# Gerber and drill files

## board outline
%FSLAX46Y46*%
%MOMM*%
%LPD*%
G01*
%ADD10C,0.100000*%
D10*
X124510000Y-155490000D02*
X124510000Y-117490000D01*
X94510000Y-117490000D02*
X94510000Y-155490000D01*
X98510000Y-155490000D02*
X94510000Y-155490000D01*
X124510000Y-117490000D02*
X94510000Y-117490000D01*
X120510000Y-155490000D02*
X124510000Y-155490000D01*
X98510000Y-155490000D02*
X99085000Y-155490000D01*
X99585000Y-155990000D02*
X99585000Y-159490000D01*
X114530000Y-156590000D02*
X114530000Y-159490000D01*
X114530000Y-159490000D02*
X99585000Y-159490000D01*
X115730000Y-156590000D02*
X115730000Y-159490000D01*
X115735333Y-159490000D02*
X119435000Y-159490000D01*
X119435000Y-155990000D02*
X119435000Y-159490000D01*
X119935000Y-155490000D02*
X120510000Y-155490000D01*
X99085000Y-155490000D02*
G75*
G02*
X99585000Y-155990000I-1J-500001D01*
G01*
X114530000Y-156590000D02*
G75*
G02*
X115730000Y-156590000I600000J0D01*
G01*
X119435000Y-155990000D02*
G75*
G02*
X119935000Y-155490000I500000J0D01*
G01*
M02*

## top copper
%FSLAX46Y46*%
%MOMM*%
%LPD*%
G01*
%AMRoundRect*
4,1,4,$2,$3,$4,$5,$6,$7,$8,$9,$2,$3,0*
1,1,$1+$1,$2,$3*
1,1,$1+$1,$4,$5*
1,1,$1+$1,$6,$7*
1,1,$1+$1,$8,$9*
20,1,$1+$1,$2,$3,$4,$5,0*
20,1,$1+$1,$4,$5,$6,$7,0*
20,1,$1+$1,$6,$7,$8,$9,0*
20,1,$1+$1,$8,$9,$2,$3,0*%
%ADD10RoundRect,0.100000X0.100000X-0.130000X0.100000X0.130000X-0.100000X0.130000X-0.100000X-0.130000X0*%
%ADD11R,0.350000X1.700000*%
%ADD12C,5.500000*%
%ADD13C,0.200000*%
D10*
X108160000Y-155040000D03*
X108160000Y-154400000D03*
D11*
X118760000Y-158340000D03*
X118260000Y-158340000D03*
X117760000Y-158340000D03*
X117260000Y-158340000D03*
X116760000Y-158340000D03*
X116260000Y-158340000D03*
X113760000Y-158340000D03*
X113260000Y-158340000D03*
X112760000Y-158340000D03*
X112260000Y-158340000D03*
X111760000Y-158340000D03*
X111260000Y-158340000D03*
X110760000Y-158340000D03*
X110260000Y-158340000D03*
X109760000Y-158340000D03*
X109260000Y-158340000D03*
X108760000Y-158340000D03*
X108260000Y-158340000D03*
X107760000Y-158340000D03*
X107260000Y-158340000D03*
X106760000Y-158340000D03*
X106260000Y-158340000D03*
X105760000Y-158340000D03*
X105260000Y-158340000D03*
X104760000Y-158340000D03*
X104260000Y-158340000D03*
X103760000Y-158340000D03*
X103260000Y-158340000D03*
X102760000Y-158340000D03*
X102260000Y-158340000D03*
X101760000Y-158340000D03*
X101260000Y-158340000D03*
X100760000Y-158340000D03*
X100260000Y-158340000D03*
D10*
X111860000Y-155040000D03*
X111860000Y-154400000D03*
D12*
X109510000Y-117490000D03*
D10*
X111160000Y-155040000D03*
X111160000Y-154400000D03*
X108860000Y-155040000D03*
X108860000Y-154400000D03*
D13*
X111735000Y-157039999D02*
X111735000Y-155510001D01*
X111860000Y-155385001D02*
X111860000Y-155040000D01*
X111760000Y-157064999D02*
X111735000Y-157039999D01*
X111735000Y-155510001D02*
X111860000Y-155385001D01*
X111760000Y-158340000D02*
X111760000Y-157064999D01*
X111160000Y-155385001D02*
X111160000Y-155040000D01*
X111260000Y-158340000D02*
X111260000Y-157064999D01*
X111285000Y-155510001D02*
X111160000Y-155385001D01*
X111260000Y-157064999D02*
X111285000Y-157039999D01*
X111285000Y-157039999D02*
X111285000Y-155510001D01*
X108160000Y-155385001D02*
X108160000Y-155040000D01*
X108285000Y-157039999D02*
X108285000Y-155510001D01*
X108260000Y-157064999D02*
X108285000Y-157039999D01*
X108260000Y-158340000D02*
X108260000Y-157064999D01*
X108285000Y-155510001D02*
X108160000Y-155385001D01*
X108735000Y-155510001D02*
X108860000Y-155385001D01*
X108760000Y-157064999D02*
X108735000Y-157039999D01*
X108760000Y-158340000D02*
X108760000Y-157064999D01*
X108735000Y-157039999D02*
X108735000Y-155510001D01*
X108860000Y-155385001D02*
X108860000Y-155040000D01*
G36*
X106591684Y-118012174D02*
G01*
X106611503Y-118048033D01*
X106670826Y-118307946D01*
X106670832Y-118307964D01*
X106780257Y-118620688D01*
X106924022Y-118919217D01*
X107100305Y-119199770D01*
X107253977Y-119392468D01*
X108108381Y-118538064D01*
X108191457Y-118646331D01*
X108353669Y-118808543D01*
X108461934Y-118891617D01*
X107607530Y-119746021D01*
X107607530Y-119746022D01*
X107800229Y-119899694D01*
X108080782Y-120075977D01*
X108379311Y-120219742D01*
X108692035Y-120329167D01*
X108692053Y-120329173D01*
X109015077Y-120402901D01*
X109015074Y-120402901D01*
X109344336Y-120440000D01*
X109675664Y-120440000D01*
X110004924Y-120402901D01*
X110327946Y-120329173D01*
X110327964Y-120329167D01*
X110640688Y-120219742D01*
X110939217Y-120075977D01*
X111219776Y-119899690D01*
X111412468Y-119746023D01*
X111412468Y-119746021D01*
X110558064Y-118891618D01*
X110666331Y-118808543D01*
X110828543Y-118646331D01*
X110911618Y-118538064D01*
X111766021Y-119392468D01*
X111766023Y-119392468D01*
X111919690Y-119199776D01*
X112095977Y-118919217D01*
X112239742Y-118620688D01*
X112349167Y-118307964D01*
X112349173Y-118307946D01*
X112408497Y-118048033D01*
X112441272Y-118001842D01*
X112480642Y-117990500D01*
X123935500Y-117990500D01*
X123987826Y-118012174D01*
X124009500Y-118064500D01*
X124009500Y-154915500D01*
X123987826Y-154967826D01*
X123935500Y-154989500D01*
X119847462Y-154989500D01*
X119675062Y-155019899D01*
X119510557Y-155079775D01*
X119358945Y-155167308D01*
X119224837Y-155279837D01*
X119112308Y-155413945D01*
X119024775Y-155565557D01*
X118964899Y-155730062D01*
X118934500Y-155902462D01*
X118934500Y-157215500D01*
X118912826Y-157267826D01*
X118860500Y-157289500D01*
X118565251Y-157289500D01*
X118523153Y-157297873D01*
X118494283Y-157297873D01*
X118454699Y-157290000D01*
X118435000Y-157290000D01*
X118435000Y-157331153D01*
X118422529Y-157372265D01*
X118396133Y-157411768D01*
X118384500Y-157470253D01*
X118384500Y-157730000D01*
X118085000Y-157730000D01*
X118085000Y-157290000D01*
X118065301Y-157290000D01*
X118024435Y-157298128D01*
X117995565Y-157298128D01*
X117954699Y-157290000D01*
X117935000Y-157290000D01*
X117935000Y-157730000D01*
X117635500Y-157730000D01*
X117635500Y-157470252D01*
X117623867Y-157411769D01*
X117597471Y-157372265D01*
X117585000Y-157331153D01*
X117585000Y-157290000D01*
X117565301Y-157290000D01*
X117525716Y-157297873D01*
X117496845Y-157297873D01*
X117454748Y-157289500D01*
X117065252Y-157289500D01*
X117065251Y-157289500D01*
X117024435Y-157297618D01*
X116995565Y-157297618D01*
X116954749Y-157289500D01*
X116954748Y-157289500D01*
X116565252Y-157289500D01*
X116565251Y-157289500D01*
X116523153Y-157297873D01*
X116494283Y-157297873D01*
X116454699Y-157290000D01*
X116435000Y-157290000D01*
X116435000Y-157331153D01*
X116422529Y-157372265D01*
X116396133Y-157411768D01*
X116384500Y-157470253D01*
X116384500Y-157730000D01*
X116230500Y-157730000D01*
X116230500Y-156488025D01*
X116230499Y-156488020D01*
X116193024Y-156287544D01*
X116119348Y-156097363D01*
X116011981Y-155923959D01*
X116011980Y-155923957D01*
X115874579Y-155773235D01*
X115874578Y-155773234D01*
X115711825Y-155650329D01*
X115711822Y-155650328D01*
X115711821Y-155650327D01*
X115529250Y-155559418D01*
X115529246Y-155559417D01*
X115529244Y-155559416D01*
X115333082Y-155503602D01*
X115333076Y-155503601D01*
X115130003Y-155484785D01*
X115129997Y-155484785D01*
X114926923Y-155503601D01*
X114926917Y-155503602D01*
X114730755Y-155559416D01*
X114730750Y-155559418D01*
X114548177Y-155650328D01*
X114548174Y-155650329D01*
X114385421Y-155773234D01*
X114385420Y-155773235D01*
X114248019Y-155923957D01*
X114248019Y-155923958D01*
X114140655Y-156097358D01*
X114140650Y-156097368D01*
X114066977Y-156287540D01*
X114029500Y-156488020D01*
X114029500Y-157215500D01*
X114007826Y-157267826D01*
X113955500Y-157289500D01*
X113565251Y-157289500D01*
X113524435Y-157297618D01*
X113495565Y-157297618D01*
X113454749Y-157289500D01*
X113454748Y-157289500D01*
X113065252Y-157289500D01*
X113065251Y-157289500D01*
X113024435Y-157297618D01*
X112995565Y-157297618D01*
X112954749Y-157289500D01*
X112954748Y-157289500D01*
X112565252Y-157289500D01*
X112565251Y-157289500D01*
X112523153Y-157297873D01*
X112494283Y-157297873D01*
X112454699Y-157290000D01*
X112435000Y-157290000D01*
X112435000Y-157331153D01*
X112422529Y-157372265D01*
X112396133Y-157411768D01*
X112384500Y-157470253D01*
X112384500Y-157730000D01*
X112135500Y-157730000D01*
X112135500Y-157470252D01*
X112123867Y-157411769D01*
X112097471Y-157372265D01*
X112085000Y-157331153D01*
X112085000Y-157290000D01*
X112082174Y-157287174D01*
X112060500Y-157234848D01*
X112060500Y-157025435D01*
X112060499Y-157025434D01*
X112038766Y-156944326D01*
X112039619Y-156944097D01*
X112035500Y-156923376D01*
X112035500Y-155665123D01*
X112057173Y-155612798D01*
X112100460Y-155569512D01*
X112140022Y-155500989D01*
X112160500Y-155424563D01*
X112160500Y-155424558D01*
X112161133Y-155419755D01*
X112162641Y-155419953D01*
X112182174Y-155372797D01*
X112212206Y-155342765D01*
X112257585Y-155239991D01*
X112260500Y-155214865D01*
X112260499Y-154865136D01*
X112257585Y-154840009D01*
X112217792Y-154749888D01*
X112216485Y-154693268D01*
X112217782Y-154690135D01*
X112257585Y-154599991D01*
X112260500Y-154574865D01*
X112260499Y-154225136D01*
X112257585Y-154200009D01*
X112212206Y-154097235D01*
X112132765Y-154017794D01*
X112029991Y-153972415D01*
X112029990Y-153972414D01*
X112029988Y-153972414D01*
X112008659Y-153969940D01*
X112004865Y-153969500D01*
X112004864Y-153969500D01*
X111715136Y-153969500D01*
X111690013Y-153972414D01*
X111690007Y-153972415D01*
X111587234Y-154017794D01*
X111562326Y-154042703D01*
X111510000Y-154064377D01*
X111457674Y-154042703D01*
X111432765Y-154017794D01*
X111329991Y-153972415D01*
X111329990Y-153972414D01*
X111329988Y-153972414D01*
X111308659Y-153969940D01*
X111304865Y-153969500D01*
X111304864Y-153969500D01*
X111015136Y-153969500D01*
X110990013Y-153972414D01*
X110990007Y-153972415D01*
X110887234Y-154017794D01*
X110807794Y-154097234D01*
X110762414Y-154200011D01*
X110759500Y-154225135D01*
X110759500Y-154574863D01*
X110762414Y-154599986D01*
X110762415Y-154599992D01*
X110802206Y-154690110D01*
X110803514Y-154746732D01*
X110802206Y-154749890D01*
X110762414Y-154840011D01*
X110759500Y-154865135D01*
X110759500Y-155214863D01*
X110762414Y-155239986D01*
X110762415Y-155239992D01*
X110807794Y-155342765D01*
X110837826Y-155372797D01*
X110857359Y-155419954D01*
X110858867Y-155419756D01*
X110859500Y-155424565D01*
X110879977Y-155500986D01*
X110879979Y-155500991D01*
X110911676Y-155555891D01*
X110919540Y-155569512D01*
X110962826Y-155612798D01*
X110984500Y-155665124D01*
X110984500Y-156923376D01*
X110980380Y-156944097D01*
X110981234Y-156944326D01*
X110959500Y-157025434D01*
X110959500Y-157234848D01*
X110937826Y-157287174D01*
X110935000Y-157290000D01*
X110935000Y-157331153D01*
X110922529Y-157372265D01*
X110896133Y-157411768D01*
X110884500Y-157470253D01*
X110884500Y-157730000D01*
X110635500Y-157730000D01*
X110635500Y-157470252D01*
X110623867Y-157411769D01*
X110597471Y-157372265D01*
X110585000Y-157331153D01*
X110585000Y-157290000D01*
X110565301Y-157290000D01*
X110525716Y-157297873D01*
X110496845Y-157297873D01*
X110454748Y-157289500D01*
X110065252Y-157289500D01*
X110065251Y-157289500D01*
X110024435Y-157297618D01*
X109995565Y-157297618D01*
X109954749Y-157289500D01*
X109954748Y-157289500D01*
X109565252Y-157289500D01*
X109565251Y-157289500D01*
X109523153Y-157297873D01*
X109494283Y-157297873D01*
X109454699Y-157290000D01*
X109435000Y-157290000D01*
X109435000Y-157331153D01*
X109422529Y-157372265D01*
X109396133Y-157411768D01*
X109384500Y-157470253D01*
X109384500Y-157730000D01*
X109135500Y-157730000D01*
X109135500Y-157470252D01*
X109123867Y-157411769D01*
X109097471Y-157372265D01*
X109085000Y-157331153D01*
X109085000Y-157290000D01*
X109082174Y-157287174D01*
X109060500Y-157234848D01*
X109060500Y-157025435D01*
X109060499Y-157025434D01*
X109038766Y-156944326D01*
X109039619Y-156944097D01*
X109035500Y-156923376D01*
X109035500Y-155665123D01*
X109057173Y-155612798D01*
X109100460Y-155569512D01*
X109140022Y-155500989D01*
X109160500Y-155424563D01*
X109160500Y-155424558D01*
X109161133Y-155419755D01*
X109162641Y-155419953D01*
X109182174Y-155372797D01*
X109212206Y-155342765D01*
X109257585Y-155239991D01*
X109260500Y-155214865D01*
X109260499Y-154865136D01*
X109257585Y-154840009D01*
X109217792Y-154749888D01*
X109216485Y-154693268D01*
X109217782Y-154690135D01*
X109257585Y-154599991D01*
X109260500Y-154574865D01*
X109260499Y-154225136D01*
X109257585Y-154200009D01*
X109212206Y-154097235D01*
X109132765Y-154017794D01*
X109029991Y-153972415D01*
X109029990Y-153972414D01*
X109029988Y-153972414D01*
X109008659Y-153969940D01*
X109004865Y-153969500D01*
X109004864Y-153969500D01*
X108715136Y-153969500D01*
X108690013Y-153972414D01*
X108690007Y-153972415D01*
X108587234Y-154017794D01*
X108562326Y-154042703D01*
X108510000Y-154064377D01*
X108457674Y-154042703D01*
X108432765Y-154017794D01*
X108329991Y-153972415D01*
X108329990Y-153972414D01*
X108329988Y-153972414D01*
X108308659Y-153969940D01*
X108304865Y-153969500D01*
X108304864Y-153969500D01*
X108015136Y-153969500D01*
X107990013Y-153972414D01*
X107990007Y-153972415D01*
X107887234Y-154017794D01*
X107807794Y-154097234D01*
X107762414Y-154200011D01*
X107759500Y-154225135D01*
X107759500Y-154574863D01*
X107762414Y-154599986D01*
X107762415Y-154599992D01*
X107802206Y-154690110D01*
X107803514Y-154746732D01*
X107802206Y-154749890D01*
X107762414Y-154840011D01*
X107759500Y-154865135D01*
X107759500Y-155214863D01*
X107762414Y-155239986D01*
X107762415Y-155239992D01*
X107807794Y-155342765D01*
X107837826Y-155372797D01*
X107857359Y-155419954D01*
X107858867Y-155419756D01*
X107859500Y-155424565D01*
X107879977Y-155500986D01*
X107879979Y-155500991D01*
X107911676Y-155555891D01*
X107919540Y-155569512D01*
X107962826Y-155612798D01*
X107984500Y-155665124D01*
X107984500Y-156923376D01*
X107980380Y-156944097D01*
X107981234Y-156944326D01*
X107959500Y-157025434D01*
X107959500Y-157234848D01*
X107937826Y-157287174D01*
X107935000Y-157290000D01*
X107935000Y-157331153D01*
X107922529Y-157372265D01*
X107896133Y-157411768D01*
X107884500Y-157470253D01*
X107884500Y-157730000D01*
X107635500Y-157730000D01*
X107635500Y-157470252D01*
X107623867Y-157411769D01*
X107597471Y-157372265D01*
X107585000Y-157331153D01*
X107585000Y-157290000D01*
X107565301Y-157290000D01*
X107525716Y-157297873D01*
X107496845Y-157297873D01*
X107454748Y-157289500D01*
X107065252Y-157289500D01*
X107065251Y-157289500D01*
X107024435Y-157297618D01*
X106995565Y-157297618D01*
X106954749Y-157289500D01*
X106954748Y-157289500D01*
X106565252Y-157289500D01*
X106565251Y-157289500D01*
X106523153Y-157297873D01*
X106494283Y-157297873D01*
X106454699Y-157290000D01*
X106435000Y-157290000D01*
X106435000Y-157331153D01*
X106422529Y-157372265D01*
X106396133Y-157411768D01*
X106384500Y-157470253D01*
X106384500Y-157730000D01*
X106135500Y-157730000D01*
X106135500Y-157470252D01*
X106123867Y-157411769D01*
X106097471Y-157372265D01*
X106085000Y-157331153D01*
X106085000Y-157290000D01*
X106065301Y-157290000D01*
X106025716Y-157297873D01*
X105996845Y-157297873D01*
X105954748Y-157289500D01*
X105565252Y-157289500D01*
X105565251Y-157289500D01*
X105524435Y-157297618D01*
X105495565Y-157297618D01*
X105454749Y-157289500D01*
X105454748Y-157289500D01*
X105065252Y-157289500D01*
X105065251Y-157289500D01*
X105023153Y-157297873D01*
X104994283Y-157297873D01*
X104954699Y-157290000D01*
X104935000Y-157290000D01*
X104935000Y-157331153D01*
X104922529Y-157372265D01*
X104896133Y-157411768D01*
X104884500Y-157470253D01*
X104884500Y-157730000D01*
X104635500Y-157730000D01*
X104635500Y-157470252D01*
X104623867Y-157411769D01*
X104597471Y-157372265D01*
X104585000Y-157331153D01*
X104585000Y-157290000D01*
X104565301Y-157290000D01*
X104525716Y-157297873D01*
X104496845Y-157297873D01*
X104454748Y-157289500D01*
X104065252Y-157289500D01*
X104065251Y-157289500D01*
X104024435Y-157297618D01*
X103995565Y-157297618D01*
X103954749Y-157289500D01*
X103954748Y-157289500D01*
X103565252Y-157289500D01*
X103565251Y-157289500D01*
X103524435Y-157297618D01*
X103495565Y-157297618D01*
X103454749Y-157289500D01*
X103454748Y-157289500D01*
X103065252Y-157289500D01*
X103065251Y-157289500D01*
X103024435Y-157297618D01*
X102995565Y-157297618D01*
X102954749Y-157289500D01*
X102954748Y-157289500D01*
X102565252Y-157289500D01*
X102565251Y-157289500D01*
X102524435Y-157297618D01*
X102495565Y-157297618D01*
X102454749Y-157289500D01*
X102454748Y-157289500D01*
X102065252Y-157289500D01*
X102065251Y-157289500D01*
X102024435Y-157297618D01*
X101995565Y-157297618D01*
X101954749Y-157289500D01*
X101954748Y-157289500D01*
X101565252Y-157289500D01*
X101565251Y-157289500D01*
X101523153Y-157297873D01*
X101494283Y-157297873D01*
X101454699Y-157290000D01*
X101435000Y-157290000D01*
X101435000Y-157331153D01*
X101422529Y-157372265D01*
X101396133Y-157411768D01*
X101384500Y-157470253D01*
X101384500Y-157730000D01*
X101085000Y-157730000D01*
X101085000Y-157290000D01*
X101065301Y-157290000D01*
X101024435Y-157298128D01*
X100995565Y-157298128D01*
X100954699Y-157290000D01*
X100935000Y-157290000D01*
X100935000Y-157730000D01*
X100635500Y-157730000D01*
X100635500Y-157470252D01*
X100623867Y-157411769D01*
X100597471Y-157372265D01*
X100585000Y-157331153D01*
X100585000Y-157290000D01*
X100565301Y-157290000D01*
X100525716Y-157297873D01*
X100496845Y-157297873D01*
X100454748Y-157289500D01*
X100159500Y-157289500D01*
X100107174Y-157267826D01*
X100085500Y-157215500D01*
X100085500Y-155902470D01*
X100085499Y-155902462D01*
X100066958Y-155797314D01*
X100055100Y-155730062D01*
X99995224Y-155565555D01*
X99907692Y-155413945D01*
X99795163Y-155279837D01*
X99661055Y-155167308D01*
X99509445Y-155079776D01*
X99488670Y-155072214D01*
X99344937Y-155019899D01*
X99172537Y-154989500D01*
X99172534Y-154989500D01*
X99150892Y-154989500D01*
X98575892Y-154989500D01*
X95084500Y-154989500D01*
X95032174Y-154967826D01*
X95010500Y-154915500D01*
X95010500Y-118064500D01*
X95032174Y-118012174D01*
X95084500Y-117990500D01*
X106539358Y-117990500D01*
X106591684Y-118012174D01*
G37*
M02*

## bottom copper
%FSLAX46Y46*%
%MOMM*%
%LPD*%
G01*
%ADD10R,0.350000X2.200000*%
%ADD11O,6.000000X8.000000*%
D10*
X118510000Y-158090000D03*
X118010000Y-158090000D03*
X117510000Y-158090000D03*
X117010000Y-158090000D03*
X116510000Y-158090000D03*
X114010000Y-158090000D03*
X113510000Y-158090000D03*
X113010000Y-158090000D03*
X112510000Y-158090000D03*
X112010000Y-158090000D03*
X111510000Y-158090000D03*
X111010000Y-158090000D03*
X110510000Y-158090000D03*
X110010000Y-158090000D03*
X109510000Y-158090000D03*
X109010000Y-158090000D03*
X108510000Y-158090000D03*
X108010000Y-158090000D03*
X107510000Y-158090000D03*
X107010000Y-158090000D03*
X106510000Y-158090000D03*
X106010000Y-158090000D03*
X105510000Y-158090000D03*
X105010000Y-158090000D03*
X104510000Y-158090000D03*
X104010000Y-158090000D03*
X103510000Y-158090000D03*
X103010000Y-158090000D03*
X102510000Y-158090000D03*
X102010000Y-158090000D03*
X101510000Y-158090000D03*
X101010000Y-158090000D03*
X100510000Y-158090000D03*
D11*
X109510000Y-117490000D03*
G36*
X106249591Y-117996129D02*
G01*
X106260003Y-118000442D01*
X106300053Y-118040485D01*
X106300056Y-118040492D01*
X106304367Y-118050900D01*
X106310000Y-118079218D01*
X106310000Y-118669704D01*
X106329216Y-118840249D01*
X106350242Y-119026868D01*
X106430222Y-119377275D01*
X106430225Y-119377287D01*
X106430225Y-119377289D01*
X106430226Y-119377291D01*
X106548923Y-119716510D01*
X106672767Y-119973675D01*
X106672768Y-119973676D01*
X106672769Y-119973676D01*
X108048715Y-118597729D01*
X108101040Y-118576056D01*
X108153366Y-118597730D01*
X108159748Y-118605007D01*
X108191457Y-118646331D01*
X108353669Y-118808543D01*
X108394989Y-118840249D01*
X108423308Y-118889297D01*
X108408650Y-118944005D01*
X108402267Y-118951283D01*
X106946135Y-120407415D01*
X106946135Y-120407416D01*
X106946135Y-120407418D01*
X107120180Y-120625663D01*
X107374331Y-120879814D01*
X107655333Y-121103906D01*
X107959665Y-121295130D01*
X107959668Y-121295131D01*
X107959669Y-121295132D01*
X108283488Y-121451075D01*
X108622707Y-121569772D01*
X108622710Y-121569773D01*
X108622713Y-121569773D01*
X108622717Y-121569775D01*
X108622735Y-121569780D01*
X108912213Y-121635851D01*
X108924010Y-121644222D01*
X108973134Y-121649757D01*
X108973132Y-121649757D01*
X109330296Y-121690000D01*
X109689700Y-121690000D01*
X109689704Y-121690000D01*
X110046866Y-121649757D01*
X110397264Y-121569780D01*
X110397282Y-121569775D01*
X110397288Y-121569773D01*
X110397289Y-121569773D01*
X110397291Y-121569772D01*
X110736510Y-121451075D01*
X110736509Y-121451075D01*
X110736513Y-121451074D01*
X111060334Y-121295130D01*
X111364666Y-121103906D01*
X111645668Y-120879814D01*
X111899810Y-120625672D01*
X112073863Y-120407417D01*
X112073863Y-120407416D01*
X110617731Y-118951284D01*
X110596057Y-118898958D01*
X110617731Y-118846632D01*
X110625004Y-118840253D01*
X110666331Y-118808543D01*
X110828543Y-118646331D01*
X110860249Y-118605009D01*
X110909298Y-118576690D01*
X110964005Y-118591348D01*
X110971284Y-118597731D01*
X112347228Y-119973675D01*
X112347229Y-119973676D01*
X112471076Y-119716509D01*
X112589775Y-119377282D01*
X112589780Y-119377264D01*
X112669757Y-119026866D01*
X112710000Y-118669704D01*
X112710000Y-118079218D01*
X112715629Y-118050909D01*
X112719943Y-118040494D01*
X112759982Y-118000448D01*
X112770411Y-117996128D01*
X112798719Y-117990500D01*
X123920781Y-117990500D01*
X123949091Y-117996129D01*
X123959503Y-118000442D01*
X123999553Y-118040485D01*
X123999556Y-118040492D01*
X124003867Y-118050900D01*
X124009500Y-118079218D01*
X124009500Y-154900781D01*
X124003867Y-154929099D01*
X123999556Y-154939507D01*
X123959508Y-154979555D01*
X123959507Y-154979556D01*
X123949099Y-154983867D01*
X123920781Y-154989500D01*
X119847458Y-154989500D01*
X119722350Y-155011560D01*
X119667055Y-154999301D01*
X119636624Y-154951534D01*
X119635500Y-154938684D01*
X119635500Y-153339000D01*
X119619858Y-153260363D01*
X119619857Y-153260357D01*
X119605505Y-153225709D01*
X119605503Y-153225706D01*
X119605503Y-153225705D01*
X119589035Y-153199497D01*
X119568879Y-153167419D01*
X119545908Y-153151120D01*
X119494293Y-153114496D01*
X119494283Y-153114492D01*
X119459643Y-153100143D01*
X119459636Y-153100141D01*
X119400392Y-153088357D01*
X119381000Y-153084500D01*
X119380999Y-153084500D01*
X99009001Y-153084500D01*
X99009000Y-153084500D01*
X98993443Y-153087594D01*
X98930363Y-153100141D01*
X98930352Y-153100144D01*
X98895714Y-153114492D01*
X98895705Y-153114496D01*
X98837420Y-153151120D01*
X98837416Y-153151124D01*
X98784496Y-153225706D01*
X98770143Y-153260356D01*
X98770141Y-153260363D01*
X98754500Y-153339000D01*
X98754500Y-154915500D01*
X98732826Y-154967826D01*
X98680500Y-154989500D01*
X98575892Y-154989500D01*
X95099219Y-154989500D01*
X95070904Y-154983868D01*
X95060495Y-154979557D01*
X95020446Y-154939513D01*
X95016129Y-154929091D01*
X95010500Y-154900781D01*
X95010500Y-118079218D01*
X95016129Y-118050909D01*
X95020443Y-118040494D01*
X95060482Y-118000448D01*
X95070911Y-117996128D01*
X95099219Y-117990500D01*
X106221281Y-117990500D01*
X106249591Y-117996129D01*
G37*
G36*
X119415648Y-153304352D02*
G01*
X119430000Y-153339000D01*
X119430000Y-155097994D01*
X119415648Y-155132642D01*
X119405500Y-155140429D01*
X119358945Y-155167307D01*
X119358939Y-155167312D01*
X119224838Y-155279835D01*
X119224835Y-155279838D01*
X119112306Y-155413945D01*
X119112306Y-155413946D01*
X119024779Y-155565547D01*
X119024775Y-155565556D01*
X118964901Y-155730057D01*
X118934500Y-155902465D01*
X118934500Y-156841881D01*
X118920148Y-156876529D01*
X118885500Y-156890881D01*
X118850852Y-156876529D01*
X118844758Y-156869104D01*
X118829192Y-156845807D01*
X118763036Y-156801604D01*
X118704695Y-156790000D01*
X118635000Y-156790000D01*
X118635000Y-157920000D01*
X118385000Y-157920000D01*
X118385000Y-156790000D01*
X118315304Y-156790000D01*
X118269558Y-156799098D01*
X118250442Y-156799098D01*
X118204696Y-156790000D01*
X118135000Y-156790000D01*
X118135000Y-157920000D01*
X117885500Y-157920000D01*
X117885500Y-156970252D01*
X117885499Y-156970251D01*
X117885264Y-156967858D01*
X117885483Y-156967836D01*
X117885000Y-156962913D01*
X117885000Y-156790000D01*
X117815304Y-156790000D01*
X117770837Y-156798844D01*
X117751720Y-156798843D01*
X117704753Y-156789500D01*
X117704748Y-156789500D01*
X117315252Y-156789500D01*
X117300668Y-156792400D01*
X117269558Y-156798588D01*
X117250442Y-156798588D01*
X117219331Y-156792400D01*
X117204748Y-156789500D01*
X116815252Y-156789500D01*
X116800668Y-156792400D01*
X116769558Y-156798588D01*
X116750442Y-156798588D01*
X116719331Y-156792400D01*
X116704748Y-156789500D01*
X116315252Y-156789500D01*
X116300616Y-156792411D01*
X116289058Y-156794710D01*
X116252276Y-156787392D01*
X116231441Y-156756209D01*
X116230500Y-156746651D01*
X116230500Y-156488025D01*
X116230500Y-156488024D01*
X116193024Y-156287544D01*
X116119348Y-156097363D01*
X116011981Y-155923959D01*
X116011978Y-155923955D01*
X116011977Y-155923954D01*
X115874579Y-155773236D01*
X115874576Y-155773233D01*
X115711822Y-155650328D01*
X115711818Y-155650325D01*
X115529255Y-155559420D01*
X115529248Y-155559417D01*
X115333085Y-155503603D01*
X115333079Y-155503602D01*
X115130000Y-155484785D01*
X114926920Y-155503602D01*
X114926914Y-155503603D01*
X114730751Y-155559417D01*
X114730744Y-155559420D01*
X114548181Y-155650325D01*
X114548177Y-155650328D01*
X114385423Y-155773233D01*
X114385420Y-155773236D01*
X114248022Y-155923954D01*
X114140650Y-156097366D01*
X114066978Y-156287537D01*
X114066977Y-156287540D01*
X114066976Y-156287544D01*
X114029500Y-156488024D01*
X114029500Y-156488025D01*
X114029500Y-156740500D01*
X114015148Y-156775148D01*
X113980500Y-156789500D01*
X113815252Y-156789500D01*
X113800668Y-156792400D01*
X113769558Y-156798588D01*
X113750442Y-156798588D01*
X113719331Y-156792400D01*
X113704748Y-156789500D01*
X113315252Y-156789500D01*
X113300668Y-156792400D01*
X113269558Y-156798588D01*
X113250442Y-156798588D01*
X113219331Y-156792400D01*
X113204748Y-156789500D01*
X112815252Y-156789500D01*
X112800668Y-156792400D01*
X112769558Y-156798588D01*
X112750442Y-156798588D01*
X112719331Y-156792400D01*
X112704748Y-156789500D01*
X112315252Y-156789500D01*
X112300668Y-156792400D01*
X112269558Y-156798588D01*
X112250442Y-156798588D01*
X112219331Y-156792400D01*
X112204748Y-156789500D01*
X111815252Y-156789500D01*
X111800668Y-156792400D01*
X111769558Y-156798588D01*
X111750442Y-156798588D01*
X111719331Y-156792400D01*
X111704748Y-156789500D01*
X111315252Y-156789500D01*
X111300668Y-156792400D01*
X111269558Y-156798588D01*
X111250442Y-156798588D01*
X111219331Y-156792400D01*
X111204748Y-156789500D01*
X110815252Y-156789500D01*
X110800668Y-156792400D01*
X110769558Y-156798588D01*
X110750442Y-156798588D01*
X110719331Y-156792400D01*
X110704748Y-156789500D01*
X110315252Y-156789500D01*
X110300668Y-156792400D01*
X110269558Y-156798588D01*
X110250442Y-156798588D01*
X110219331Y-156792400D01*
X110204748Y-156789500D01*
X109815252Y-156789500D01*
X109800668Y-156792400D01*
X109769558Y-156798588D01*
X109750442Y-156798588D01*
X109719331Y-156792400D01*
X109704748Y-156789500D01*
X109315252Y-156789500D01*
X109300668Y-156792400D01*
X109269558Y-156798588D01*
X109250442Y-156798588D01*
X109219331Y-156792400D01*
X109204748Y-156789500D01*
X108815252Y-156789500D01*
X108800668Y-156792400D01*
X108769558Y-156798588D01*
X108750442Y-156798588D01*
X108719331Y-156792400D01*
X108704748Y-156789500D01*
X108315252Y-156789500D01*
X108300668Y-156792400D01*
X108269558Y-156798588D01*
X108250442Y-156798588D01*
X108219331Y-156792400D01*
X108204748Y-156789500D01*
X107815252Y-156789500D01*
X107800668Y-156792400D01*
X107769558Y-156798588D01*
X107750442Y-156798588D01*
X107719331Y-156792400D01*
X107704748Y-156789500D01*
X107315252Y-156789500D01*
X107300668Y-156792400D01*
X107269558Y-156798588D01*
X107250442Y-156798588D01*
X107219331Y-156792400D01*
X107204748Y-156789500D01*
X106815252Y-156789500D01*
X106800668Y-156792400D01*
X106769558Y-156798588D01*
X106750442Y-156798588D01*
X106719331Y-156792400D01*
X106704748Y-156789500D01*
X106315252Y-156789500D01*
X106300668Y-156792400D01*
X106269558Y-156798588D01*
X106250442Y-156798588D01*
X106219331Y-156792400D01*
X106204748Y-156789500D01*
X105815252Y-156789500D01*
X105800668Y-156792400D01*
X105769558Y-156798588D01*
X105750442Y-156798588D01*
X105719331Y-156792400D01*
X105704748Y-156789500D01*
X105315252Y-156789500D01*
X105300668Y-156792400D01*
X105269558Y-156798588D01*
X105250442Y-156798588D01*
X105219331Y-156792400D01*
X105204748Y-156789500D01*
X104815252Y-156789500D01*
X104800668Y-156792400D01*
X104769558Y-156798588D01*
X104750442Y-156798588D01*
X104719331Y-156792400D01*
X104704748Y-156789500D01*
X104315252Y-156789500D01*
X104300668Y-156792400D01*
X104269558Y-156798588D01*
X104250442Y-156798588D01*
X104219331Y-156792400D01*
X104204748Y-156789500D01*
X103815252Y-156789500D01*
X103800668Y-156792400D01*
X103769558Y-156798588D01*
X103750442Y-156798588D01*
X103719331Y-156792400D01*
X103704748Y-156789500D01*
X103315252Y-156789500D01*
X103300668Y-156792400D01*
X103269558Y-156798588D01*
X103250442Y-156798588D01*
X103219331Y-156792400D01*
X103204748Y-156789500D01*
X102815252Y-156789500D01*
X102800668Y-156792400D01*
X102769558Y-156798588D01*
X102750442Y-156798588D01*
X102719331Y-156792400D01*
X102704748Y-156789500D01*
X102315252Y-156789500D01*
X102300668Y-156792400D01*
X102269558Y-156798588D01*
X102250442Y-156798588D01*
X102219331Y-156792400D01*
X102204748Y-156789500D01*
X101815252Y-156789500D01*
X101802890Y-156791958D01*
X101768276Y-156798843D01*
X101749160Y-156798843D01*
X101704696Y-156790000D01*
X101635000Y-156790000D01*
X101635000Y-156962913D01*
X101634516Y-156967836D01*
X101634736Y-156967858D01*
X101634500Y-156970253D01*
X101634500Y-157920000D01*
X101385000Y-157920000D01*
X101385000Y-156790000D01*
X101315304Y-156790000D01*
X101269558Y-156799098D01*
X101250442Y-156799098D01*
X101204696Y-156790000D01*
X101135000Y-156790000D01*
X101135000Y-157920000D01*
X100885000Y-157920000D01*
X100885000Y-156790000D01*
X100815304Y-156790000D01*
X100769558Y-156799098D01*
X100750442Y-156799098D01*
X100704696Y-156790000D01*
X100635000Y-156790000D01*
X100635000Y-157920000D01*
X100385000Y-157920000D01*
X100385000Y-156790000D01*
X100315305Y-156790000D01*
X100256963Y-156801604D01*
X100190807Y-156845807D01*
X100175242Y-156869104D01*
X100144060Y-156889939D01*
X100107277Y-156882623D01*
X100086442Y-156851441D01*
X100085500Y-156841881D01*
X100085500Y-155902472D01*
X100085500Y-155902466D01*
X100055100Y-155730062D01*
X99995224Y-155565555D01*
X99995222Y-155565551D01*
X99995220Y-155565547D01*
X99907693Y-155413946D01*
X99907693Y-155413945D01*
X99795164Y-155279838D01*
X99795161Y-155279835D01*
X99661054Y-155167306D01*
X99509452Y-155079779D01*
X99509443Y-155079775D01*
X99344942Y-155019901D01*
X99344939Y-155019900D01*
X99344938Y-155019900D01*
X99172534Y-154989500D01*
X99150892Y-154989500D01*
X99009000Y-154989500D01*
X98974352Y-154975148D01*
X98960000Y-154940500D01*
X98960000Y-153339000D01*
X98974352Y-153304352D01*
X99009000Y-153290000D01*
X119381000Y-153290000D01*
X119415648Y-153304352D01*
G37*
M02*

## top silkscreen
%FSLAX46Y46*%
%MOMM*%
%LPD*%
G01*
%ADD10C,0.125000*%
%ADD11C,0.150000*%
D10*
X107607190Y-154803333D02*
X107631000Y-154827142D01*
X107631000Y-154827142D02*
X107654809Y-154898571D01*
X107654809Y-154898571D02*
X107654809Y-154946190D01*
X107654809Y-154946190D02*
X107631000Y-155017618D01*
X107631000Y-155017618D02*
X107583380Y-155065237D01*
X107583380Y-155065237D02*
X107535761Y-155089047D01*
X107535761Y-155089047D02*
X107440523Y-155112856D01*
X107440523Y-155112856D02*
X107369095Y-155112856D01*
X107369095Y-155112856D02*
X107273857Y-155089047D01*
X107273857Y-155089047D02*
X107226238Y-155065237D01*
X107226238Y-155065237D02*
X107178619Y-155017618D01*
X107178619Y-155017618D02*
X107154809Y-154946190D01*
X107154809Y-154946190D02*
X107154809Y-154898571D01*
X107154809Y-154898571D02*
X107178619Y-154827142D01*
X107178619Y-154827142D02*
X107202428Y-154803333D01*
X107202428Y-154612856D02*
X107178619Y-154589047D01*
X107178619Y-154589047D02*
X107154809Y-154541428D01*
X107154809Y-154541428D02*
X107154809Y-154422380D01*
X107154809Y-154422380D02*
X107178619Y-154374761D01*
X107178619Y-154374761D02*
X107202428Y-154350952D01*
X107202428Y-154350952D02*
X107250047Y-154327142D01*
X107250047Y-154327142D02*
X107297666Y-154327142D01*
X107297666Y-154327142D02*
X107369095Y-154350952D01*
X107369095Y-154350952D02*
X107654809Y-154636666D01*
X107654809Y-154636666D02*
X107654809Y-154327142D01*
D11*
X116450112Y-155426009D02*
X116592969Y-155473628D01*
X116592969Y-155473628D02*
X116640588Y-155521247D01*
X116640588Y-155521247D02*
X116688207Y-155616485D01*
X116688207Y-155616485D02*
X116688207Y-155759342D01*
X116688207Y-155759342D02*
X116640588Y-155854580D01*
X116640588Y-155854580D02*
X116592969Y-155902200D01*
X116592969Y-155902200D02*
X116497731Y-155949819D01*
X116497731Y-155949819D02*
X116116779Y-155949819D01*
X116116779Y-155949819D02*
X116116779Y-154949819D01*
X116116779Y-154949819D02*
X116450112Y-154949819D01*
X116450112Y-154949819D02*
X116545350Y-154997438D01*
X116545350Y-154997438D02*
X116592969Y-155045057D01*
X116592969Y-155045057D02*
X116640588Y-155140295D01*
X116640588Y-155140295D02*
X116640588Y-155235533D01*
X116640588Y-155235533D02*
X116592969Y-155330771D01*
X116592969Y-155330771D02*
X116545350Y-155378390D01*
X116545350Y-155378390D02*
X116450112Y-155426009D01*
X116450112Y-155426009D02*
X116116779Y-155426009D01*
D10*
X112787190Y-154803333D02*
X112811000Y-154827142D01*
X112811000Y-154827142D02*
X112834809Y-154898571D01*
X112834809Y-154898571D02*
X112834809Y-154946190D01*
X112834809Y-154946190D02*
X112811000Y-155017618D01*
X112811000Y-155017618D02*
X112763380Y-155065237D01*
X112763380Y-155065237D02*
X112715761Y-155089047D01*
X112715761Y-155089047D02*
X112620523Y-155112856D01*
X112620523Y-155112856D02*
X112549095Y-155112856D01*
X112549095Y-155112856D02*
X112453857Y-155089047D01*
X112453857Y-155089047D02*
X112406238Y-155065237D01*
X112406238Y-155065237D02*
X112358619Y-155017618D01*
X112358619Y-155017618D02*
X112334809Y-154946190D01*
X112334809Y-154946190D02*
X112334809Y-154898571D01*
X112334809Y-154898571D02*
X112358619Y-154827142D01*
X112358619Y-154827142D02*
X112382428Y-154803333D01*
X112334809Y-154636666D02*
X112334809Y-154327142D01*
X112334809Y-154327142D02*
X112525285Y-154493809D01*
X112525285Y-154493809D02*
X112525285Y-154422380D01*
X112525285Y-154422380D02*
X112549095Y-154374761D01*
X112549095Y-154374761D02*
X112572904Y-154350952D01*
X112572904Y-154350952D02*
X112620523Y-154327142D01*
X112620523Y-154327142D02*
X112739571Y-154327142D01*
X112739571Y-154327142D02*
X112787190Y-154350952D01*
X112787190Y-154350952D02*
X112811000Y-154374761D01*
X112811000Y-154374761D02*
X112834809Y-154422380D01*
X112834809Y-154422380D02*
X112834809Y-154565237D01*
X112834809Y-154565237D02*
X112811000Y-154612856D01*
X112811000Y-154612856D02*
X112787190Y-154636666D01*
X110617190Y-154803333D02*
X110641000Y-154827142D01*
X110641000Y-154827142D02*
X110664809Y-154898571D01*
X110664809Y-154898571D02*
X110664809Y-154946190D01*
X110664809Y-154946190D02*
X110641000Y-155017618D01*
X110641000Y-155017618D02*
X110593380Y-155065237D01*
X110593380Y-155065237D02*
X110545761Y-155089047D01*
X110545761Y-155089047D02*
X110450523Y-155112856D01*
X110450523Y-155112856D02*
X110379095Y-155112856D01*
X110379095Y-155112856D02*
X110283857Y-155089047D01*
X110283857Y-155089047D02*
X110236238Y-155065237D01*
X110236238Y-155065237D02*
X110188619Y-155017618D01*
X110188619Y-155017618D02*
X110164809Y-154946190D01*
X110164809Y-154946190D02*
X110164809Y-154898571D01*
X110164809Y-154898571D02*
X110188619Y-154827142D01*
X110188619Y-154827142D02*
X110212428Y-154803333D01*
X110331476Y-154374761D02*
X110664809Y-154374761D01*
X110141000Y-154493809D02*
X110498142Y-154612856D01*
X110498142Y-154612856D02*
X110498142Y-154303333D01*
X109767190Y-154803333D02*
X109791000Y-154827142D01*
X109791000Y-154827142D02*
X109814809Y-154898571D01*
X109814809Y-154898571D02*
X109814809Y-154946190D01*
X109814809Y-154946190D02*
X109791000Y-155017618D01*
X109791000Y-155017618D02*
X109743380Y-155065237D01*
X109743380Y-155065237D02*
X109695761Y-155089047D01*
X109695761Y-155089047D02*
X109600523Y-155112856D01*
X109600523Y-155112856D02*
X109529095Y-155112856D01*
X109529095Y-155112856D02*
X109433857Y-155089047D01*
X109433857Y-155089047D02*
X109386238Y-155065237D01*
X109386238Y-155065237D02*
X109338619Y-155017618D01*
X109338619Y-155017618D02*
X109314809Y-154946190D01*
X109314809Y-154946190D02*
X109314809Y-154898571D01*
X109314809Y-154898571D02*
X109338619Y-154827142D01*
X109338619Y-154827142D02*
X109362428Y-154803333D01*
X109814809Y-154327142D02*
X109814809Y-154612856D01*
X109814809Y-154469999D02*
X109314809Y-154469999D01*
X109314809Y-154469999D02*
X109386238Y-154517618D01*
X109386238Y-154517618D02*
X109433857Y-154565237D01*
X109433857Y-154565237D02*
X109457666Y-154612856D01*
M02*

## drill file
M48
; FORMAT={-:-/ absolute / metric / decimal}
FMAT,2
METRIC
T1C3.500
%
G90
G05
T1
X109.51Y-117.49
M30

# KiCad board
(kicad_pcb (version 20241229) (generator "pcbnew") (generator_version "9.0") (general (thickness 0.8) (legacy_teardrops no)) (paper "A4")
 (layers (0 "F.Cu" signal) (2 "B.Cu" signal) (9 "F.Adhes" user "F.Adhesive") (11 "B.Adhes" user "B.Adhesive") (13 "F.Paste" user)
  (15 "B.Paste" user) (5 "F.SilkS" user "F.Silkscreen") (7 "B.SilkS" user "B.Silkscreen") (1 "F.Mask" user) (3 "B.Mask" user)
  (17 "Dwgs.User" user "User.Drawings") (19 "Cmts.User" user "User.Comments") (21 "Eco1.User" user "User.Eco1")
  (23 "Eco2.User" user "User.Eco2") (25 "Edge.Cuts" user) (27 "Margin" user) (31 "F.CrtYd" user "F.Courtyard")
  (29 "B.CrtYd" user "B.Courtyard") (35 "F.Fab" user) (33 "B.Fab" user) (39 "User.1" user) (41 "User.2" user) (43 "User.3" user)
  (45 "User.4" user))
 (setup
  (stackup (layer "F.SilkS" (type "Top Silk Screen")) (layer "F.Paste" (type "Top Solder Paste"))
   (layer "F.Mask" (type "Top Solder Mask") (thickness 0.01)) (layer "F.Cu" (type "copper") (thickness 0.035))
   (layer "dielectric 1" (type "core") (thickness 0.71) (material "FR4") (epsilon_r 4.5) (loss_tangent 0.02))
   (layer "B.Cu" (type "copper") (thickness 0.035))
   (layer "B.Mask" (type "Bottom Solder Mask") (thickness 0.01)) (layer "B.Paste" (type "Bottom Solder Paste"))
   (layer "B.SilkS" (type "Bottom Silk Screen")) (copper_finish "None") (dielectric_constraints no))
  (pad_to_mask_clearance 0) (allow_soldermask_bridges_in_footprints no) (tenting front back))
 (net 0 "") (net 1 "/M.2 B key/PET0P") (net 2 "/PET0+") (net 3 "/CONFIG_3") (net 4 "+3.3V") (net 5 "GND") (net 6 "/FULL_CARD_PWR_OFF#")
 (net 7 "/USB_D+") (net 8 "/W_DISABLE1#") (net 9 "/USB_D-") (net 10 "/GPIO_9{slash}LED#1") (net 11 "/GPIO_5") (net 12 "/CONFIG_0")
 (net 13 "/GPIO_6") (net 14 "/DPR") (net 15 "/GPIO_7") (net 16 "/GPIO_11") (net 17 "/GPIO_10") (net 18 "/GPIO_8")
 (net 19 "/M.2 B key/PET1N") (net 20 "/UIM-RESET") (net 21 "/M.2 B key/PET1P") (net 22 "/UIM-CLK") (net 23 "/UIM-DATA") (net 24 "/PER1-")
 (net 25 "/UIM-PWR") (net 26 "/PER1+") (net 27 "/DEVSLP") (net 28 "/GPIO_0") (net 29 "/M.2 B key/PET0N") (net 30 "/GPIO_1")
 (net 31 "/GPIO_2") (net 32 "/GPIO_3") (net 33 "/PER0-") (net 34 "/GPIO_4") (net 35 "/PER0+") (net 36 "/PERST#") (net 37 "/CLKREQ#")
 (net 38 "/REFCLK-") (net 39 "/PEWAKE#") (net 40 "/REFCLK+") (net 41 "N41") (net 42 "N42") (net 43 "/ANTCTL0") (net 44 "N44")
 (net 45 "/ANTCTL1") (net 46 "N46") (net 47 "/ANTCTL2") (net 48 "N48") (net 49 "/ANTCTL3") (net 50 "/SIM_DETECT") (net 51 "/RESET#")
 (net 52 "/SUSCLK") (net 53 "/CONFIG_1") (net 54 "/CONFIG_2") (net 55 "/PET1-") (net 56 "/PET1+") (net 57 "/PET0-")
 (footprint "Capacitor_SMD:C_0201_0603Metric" (layer "F.Cu") (at 108.16 154.72 90)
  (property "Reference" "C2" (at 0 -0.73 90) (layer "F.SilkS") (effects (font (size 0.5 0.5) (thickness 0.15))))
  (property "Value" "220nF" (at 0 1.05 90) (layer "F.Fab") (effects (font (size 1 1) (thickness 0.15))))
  (pad "" smd roundrect (at -0.345 0 90) (size 0.318 0.36) (layers "F.Paste") (roundrect_rratio 0.25))
  (pad "" smd roundrect (at 0.345 0 90) (size 0.318 0.36) (layers "F.Paste") (roundrect_rratio 0.25))
  (pad "1" smd roundrect (at -0.32 0 90) (size 0.46 0.4) (layers "F.Cu" "F.Mask") (roundrect_rratio 0.25) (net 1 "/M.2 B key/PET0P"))
  (pad "2" smd roundrect (at 0.32 0 90) (size 0.46 0.4) (layers "F.Cu" "F.Mask") (roundrect_rratio 0.25) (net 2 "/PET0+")))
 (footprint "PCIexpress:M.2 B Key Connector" (layer "F.Cu") (at 109.51 158.38)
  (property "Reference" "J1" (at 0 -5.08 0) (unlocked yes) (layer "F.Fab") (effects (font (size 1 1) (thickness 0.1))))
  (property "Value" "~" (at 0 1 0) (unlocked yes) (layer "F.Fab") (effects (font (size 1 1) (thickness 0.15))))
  (fp_line (start -11 -2.89) (end -10.425 -2.89) (stroke (width 0.1) (type default)) (layer "Edge.Cuts"))
  (fp_line (start -9.925 -2.39) (end -9.925 1.11) (stroke (width 0.1) (type default)) (layer "Edge.Cuts"))
  (fp_line (start 5.02 -1.79) (end 5.02 1.11) (stroke (width 0.1) (type default)) (layer "Edge.Cuts"))
  (fp_line (start 5.02 1.11) (end -9.925 1.11) (stroke (width 0.1) (type default)) (layer "Edge.Cuts"))
  (fp_line (start 6.22 -1.79) (end 6.22 1.11) (stroke (width 0.1) (type default)) (layer "Edge.Cuts"))
  (fp_line (start 6.225333 1.11) (end 9.925 1.11) (stroke (width 0.1) (type default)) (layer "Edge.Cuts"))
  (fp_line (start 9.925 -2.39) (end 9.925 1.11) (stroke (width 0.1) (type default)) (layer "Edge.Cuts"))
  (fp_line (start 10.425 -2.89) (end 11 -2.89) (stroke (width 0.1) (type default)) (layer "Edge.Cuts"))
  (fp_arc (start -10.425 -2.89) (mid -10.071447 -2.743553) (end -9.925 -2.39) (stroke (width 0.1) (type default)) (layer "Edge.Cuts"))
  (fp_arc (start 5.02 -1.79) (mid 5.62 -2.39) (end 6.22 -1.79) (stroke (width 0.1) (type default)) (layer "Edge.Cuts"))
  (fp_arc (start 9.925 -2.39) (mid 10.071447 -2.743553) (end 10.425 -2.89) (stroke (width 0.1) (type default)) (layer "Edge.Cuts"))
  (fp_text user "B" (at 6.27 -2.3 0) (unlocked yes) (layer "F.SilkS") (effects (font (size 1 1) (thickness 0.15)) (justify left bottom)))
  (pad "1" smd rect (at 9.25 -0.04 180) (size 0.35 1.7) (layers "F.Cu") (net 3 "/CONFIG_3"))
  (pad "2" smd rect (at 9 -0.29 180) (size 0.35 2.2) (layers "B.Cu") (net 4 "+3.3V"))
  (pad "3" smd rect (at 8.75 -0.04 180) (size 0.35 1.7) (layers "F.Cu") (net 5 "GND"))
  (pad "4" smd rect (at 8.5 -0.29 180) (size 0.35 2.2) (layers "B.Cu") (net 4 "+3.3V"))
  (pad "5" smd rect (at 8.25 -0.04 180) (size 0.35 1.7) (layers "F.Cu") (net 5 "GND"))
  (pad "6" smd rect (at 8 -0.29 180) (size 0.35 2.2) (layers "B.Cu") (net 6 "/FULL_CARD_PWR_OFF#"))
  (pad "7" smd rect (at 7.75 -0.04 180) (size 0.35 1.7) (layers "F.Cu") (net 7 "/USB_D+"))
  (pad "8" smd rect (at 7.5 -0.29 180) (size 0.35 2.2) (layers "B.Cu") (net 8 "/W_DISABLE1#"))
  (pad "9" smd rect (at 7.25 -0.04 180) (size 0.35 1.7) (layers "F.Cu") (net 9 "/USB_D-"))
  (pad "10" smd rect (at 7 -0.29 180) (size 0.35 2.2) (layers "B.Cu") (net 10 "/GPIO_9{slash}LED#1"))
  (pad "11" smd rect (at 6.75 -0.04 180) (size 0.35 1.7) (layers "F.Cu") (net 5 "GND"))
  (pad "20" smd rect (at 4.5 -0.29 180) (size 0.35 2.2) (layers "B.Cu") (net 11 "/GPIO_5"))
  (pad "21" smd rect (at 4.25 -0.04 180) (size 0.35 1.7) (layers "F.Cu") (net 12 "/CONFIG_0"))
  (pad "22" smd rect (at 4 -0.29 180) (size 0.35 2.2) (layers "B.Cu") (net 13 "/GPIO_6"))
  (pad "23" smd rect (at 3.75 -0.04 180) (size 0.35 1.7) (layers "F.Cu") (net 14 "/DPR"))
  (pad "24" smd rect (at 3.5 -0.29 180) (size 0.35 2.2) (layers "B.Cu") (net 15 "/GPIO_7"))
  (pad "25" smd rect (at 3.25 -0.04 180) (size 0.35 1.7) (layers "F.Cu") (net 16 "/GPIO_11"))
  (pad "26" smd rect (at 3 -0.29 180) (size 0.35 2.2) (layers "B.Cu") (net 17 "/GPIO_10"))
  (pad "27" smd rect (at 2.75 -0.04 180) (size 0.35 1.7) (layers "F.Cu") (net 5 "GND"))
  (pad "28" smd rect (at 2.5 -0.29 180) (size 0.35 2.2) (layers "B.Cu") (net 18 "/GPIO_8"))
  (pad "29" smd rect (at 2.25 -0.04 180) (size 0.35 1.7) (layers "F.Cu") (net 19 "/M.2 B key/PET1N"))
  (pad "30" smd rect (at 2 -0.29 180) (size 0.35 2.2) (layers "B.Cu") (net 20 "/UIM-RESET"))
  (pad "31" smd rect (at 1.75 -0.04 180) (size 0.35 1.7) (layers "F.Cu") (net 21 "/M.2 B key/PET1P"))
  (pad "32" smd rect (at 1.5 -0.29 180) (size 0.35 2.2) (layers "B.Cu") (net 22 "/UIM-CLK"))
  (pad "33" smd rect (at 1.25 -0.04 180) (size 0.35 1.7) (layers "F.Cu") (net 5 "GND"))
  (pad "34" smd rect (at 1 -0.29 180) (size 0.35 2.2) (layers "B.Cu") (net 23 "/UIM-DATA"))
  (pad "35" smd rect (at 0.75 -0.04 180) (size 0.35 1.7) (layers "F.Cu") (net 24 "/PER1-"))
  (pad "36" smd rect (at 0.5 -0.29 180) (size 0.35 2.2) (layers "B.Cu") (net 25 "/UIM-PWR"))
  (pad "37" smd rect (at 0.25 -0.04 180) (size 0.35 1.7) (layers "F.Cu") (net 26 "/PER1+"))
  (pad "38" smd rect (at 0 -0.29 180) (size 0.35 2.2) (layers "B.Cu") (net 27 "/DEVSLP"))
  (pad "39" smd rect (at -0.25 -0.04 180) (size 0.35 1.7) (layers "F.Cu") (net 5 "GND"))
  (pad "40" smd rect (at -0.5 -0.29 180) (size 0.35 2.2) (layers "B.Cu") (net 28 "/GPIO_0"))
  (pad "41" smd rect (at -0.75 -0.04 180) (size 0.35 1.7) (layers "F.Cu") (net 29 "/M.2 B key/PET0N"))
  (pad "42" smd rect (at -1 -0.29 180) (size 0.35 2.2) (layers "B.Cu") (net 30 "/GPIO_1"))
  (pad "43" smd rect (at -1.25 -0.04 180) (size 0.35 1.7) (layers "F.Cu") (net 1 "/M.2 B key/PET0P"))
  (pad "44" smd rect (at -1.5 -0.29 180) (size 0.35 2.2) (layers "B.Cu") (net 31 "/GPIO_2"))
  (pad "45" smd rect (at -1.75 -0.04 180) (size 0.35 1.7) (layers "F.Cu") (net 5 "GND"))
  (pad "46" smd rect (at -2 -0.29 180) (size 0.35 2.2) (layers "B.Cu") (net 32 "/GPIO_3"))
  (pad "47" smd rect (at -2.25 -0.04 180) (size 0.35 1.7) (layers "F.Cu") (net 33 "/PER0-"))
  (pad "48" smd rect (at -2.5 -0.29 180) (size 0.35 2.2) (layers "B.Cu") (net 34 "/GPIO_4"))
  (pad "49" smd rect (at -2.75 -0.04 180) (size 0.35 1.7) (layers "F.Cu") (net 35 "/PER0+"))
  (pad "50" smd rect (at -3 -0.29 180) (size 0.35 2.2) (layers "B.Cu") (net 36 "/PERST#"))
  (pad "51" smd rect (at -3.25 -0.04 180) (size 0.35 1.7) (layers "F.Cu") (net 5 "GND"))
  (pad "52" smd rect (at -3.5 -0.29 180) (size 0.35 2.2) (layers "B.Cu") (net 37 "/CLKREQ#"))
  (pad "53" smd rect (at -3.75 -0.04 180) (size 0.35 1.7) (layers "F.Cu") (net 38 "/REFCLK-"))
  (pad "54" smd rect (at -4 -0.29 180) (size 0.35 2.2) (layers "B.Cu") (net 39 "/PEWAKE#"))
  (pad "55" smd rect (at -4.25 -0.04 180) (size 0.35 1.7) (layers "F.Cu") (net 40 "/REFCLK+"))
  (pad "56" smd rect (at -4.5 -0.29 180) (size 0.35 2.2) (layers "B.Cu") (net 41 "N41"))
  (pad "57" smd rect (at -4.75 -0.04 180) (size 0.35 1.7) (layers "F.Cu") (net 5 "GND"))
  (pad "58" smd rect (at -5 -0.29 180) (size 0.35 2.2) (layers "B.Cu") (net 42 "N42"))
  (pad "59" smd rect (at -5.25 -0.04 180) (size 0.35 1.7) (layers "F.Cu") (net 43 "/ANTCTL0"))
  (pad "60" smd rect (at -5.5 -0.29 180) (size 0.35 2.2) (layers "B.Cu") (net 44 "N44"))
  (pad "61" smd rect (at -5.75 -0.04 180) (size 0.35 1.7) (layers "F.Cu") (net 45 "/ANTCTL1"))
  (pad "62" smd rect (at -6 -0.29 180) (size 0.35 2.2) (layers "B.Cu") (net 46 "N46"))
  (pad "63" smd rect (at -6.25 -0.04 180) (size 0.35 1.7) (layers "F.Cu") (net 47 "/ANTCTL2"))
  (pad "64" smd rect (at -6.5 -0.29 180) (size 0.35 2.2) (layers "B.Cu") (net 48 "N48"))
  (pad "65" smd rect (at -6.75 -0.04 180) (size 0.35 1.7) (layers "F.Cu") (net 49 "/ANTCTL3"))
  (pad "66" smd rect (at -7 -0.29 180) (size 0.35 2.2) (layers "B.Cu") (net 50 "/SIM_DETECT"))
  (pad "67" smd rect (at -7.25 -0.04 180) (size 0.35 1.7) (layers "F.Cu") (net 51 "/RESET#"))
  (pad "68" smd rect (at -7.5 -0.29 180) (size 0.35 2.2) (layers "B.Cu") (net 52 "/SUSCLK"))
  (pad "69" smd rect (at -7.75 -0.04 180) (size 0.35 1.7) (layers "F.Cu") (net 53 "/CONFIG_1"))
  (pad "70" smd rect (at -8 -0.29 180) (size 0.35 2.2) (layers "B.Cu") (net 4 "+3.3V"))
  (pad "71" smd rect (at -8.25 -0.04 180) (size 0.35 1.7) (layers "F.Cu") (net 5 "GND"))
  (pad "72" smd rect (at -8.5 -0.29 180) (size 0.35 2.2) (layers "B.Cu") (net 4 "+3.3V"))
  (pad "73" smd rect (at -8.75 -0.04 180) (size 0.35 1.7) (layers "F.Cu") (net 5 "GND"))
  (pad "74" smd rect (at -9 -0.29 180) (size 0.35 2.2) (layers "B.Cu") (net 4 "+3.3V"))
  (pad "75" smd rect (at -9.25 -0.04 180) (size 0.35 1.7) (layers "F.Cu") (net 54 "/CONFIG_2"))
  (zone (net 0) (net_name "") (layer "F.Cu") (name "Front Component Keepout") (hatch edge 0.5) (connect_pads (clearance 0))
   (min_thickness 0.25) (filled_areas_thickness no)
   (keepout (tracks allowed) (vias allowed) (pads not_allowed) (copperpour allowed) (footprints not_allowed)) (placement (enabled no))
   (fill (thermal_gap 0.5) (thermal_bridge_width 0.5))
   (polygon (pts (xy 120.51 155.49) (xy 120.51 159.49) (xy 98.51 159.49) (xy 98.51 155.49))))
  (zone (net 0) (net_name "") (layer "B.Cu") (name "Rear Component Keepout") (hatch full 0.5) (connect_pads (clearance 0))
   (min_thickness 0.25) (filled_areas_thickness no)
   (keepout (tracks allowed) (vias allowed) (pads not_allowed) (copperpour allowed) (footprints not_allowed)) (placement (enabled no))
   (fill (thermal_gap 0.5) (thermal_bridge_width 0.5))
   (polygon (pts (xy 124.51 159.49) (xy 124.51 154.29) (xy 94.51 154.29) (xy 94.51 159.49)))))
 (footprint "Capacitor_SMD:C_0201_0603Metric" (layer "F.Cu") (at 111.86 154.72 90)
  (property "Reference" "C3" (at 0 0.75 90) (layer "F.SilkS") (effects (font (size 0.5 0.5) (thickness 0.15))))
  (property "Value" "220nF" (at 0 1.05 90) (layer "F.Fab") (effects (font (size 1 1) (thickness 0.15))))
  (pad "" smd roundrect (at -0.345 0 90) (size 0.318 0.36) (layers "F.Paste") (roundrect_rratio 0.25))
  (pad "" smd roundrect (at 0.345 0 90) (size 0.318 0.36) (layers "F.Paste") (roundrect_rratio 0.25))
  (pad "1" smd roundrect (at -0.32 0 90) (size 0.46 0.4) (layers "F.Cu" "F.Mask") (roundrect_rratio 0.25) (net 19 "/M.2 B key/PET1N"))
  (pad "2" smd roundrect (at 0.32 0 90) (size 0.46 0.4) (layers "F.Cu" "F.Mask") (roundrect_rratio 0.25) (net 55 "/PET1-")))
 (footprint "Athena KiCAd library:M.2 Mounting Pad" (layer "F.Cu") (at 109.51 117.49)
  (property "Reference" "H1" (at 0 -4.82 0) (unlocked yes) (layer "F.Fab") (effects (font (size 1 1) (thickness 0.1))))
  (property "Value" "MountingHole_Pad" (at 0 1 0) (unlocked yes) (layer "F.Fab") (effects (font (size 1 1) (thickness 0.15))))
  (pad "1" thru_hole circle (at 0 0) (size 5.5 5.5) (drill 3.5) (layers "*.Cu" "*.Mask") (remove_unused_layers no) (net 5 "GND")
   (padstack (mode front_inner_back)
    (layer "Inner" (shape circle) (size 5.5 5.5) (zone_connect -1))
    (layer "B.Cu" (shape oval) (size 6 8) (thermal_bridge_angle 45) (zone_connect -1)))))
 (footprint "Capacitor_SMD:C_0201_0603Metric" (layer "F.Cu") (at 111.16 154.72 90)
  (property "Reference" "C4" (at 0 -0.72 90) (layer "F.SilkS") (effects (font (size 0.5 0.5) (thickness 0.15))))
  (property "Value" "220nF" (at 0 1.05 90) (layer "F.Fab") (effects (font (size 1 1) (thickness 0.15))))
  (pad "" smd roundrect (at -0.345 0 90) (size 0.318 0.36) (layers "F.Paste") (roundrect_rratio 0.25))
  (pad "" smd roundrect (at 0.345 0 90) (size 0.318 0.36) (layers "F.Paste") (roundrect_rratio 0.25))
  (pad "1" smd roundrect (at -0.32 0 90) (size 0.46 0.4) (layers "F.Cu" "F.Mask") (roundrect_rratio 0.25) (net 21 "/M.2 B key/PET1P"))
  (pad "2" smd roundrect (at 0.32 0 90) (size 0.46 0.4) (layers "F.Cu" "F.Mask") (roundrect_rratio 0.25) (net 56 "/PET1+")))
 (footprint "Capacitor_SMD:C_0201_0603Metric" (layer "F.Cu") (at 108.86 154.72 90)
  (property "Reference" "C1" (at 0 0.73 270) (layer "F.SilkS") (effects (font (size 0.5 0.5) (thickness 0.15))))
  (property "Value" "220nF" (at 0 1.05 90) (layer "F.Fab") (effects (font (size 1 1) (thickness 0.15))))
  (pad "" smd roundrect (at -0.345 0 90) (size 0.318 0.36) (layers "F.Paste") (roundrect_rratio 0.25))
  (pad "" smd roundrect (at 0.345 0 90) (size 0.318 0.36) (layers "F.Paste") (roundrect_rratio 0.25))
  (pad "1" smd roundrect (at -0.32 0 90) (size 0.46 0.4) (layers "F.Cu" "F.Mask") (roundrect_rratio 0.25) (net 29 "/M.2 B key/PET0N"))
  (pad "2" smd roundrect (at 0.32 0 90) (size 0.46 0.4) (layers "F.Cu" "F.Mask") (roundrect_rratio 0.25) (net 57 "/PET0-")))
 (gr_line (start 124.51 155.49) (end 124.51 117.49) (stroke (width 0.1) (type default)) (layer "Edge.Cuts"))
 (gr_line (start 94.51 117.49) (end 94.51 155.49) (stroke (width 0.1) (type default)) (layer "Edge.Cuts"))
 (gr_line (start 98.51 155.49) (end 94.51 155.49) (stroke (width 0.1) (type default)) (layer "Edge.Cuts"))
 (gr_line (start 124.51 117.49) (end 94.51 117.49) (stroke (width 0.1) (type default)) (layer "Edge.Cuts"))
 (gr_line (start 120.51 155.49) (end 124.51 155.49) (stroke (width 0.1) (type default)) (layer "Edge.Cuts"))
 (segment (start 111.735 157.039999) (end 111.735 155.510001) (width 0.2) (layer "F.Cu") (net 19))
 (segment (start 111.86 155.385001) (end 111.86 155.04) (width 0.2) (layer "F.Cu") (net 19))
 (segment (start 111.76 157.064999) (end 111.735 157.039999) (width 0.2) (layer "F.Cu") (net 19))
 (segment (start 111.735 155.510001) (end 111.86 155.385001) (width 0.2) (layer "F.Cu") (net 19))
 (segment (start 111.76 158.34) (end 111.76 157.064999) (width 0.2) (layer "F.Cu") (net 19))
 (segment (start 111.16 155.385001) (end 111.16 155.04) (width 0.2) (layer "F.Cu") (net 21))
 (segment (start 111.26 158.34) (end 111.26 157.064999) (width 0.2) (layer "F.Cu") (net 21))
 (segment (start 111.285 155.510001) (end 111.16 155.385001) (width 0.2) (layer "F.Cu") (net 21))
 (segment (start 111.26 157.064999) (end 111.285 157.039999) (width 0.2) (layer "F.Cu") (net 21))
 (segment (start 111.285 157.039999) (end 111.285 155.510001) (width 0.2) (layer "F.Cu") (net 21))
 (segment (start 108.16 155.385001) (end 108.16 155.04) (width 0.2) (layer "F.Cu") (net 1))
 (segment (start 108.285 157.039999) (end 108.285 155.510001) (width 0.2) (layer "F.Cu") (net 1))
 (segment (start 108.26 157.064999) (end 108.285 157.039999) (width 0.2) (layer "F.Cu") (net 1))
 (segment (start 108.26 158.34) (end 108.26 157.064999) (width 0.2) (layer "F.Cu") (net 1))
 (segment (start 108.285 155.510001) (end 108.16 155.385001) (width 0.2) (layer "F.Cu") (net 1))
 (segment (start 108.735 155.510001) (end 108.86 155.385001) (width 0.2) (layer "F.Cu") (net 29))
 (segment (start 108.76 157.064999) (end 108.735 157.039999) (width 0.2) (layer "F.Cu") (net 29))
 (segment (start 108.76 158.34) (end 108.76 157.064999) (width 0.2) (layer "F.Cu") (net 29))
 (segment (start 108.735 157.039999) (end 108.735 155.510001) (width 0.2) (layer "F.Cu") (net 29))
 (segment (start 108.86 155.385001) (end 108.86 155.04) (width 0.2) (layer "F.Cu") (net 29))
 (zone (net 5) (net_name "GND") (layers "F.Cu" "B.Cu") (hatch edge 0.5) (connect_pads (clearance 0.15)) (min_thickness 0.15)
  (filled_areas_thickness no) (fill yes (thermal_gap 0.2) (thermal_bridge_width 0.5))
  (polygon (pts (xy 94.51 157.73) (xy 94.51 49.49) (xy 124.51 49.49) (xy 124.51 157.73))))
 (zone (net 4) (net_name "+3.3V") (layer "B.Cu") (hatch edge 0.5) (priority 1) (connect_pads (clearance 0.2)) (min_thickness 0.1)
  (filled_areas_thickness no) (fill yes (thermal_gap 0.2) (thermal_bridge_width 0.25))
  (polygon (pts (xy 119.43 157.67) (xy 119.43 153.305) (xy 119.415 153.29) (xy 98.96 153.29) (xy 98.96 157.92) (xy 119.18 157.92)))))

